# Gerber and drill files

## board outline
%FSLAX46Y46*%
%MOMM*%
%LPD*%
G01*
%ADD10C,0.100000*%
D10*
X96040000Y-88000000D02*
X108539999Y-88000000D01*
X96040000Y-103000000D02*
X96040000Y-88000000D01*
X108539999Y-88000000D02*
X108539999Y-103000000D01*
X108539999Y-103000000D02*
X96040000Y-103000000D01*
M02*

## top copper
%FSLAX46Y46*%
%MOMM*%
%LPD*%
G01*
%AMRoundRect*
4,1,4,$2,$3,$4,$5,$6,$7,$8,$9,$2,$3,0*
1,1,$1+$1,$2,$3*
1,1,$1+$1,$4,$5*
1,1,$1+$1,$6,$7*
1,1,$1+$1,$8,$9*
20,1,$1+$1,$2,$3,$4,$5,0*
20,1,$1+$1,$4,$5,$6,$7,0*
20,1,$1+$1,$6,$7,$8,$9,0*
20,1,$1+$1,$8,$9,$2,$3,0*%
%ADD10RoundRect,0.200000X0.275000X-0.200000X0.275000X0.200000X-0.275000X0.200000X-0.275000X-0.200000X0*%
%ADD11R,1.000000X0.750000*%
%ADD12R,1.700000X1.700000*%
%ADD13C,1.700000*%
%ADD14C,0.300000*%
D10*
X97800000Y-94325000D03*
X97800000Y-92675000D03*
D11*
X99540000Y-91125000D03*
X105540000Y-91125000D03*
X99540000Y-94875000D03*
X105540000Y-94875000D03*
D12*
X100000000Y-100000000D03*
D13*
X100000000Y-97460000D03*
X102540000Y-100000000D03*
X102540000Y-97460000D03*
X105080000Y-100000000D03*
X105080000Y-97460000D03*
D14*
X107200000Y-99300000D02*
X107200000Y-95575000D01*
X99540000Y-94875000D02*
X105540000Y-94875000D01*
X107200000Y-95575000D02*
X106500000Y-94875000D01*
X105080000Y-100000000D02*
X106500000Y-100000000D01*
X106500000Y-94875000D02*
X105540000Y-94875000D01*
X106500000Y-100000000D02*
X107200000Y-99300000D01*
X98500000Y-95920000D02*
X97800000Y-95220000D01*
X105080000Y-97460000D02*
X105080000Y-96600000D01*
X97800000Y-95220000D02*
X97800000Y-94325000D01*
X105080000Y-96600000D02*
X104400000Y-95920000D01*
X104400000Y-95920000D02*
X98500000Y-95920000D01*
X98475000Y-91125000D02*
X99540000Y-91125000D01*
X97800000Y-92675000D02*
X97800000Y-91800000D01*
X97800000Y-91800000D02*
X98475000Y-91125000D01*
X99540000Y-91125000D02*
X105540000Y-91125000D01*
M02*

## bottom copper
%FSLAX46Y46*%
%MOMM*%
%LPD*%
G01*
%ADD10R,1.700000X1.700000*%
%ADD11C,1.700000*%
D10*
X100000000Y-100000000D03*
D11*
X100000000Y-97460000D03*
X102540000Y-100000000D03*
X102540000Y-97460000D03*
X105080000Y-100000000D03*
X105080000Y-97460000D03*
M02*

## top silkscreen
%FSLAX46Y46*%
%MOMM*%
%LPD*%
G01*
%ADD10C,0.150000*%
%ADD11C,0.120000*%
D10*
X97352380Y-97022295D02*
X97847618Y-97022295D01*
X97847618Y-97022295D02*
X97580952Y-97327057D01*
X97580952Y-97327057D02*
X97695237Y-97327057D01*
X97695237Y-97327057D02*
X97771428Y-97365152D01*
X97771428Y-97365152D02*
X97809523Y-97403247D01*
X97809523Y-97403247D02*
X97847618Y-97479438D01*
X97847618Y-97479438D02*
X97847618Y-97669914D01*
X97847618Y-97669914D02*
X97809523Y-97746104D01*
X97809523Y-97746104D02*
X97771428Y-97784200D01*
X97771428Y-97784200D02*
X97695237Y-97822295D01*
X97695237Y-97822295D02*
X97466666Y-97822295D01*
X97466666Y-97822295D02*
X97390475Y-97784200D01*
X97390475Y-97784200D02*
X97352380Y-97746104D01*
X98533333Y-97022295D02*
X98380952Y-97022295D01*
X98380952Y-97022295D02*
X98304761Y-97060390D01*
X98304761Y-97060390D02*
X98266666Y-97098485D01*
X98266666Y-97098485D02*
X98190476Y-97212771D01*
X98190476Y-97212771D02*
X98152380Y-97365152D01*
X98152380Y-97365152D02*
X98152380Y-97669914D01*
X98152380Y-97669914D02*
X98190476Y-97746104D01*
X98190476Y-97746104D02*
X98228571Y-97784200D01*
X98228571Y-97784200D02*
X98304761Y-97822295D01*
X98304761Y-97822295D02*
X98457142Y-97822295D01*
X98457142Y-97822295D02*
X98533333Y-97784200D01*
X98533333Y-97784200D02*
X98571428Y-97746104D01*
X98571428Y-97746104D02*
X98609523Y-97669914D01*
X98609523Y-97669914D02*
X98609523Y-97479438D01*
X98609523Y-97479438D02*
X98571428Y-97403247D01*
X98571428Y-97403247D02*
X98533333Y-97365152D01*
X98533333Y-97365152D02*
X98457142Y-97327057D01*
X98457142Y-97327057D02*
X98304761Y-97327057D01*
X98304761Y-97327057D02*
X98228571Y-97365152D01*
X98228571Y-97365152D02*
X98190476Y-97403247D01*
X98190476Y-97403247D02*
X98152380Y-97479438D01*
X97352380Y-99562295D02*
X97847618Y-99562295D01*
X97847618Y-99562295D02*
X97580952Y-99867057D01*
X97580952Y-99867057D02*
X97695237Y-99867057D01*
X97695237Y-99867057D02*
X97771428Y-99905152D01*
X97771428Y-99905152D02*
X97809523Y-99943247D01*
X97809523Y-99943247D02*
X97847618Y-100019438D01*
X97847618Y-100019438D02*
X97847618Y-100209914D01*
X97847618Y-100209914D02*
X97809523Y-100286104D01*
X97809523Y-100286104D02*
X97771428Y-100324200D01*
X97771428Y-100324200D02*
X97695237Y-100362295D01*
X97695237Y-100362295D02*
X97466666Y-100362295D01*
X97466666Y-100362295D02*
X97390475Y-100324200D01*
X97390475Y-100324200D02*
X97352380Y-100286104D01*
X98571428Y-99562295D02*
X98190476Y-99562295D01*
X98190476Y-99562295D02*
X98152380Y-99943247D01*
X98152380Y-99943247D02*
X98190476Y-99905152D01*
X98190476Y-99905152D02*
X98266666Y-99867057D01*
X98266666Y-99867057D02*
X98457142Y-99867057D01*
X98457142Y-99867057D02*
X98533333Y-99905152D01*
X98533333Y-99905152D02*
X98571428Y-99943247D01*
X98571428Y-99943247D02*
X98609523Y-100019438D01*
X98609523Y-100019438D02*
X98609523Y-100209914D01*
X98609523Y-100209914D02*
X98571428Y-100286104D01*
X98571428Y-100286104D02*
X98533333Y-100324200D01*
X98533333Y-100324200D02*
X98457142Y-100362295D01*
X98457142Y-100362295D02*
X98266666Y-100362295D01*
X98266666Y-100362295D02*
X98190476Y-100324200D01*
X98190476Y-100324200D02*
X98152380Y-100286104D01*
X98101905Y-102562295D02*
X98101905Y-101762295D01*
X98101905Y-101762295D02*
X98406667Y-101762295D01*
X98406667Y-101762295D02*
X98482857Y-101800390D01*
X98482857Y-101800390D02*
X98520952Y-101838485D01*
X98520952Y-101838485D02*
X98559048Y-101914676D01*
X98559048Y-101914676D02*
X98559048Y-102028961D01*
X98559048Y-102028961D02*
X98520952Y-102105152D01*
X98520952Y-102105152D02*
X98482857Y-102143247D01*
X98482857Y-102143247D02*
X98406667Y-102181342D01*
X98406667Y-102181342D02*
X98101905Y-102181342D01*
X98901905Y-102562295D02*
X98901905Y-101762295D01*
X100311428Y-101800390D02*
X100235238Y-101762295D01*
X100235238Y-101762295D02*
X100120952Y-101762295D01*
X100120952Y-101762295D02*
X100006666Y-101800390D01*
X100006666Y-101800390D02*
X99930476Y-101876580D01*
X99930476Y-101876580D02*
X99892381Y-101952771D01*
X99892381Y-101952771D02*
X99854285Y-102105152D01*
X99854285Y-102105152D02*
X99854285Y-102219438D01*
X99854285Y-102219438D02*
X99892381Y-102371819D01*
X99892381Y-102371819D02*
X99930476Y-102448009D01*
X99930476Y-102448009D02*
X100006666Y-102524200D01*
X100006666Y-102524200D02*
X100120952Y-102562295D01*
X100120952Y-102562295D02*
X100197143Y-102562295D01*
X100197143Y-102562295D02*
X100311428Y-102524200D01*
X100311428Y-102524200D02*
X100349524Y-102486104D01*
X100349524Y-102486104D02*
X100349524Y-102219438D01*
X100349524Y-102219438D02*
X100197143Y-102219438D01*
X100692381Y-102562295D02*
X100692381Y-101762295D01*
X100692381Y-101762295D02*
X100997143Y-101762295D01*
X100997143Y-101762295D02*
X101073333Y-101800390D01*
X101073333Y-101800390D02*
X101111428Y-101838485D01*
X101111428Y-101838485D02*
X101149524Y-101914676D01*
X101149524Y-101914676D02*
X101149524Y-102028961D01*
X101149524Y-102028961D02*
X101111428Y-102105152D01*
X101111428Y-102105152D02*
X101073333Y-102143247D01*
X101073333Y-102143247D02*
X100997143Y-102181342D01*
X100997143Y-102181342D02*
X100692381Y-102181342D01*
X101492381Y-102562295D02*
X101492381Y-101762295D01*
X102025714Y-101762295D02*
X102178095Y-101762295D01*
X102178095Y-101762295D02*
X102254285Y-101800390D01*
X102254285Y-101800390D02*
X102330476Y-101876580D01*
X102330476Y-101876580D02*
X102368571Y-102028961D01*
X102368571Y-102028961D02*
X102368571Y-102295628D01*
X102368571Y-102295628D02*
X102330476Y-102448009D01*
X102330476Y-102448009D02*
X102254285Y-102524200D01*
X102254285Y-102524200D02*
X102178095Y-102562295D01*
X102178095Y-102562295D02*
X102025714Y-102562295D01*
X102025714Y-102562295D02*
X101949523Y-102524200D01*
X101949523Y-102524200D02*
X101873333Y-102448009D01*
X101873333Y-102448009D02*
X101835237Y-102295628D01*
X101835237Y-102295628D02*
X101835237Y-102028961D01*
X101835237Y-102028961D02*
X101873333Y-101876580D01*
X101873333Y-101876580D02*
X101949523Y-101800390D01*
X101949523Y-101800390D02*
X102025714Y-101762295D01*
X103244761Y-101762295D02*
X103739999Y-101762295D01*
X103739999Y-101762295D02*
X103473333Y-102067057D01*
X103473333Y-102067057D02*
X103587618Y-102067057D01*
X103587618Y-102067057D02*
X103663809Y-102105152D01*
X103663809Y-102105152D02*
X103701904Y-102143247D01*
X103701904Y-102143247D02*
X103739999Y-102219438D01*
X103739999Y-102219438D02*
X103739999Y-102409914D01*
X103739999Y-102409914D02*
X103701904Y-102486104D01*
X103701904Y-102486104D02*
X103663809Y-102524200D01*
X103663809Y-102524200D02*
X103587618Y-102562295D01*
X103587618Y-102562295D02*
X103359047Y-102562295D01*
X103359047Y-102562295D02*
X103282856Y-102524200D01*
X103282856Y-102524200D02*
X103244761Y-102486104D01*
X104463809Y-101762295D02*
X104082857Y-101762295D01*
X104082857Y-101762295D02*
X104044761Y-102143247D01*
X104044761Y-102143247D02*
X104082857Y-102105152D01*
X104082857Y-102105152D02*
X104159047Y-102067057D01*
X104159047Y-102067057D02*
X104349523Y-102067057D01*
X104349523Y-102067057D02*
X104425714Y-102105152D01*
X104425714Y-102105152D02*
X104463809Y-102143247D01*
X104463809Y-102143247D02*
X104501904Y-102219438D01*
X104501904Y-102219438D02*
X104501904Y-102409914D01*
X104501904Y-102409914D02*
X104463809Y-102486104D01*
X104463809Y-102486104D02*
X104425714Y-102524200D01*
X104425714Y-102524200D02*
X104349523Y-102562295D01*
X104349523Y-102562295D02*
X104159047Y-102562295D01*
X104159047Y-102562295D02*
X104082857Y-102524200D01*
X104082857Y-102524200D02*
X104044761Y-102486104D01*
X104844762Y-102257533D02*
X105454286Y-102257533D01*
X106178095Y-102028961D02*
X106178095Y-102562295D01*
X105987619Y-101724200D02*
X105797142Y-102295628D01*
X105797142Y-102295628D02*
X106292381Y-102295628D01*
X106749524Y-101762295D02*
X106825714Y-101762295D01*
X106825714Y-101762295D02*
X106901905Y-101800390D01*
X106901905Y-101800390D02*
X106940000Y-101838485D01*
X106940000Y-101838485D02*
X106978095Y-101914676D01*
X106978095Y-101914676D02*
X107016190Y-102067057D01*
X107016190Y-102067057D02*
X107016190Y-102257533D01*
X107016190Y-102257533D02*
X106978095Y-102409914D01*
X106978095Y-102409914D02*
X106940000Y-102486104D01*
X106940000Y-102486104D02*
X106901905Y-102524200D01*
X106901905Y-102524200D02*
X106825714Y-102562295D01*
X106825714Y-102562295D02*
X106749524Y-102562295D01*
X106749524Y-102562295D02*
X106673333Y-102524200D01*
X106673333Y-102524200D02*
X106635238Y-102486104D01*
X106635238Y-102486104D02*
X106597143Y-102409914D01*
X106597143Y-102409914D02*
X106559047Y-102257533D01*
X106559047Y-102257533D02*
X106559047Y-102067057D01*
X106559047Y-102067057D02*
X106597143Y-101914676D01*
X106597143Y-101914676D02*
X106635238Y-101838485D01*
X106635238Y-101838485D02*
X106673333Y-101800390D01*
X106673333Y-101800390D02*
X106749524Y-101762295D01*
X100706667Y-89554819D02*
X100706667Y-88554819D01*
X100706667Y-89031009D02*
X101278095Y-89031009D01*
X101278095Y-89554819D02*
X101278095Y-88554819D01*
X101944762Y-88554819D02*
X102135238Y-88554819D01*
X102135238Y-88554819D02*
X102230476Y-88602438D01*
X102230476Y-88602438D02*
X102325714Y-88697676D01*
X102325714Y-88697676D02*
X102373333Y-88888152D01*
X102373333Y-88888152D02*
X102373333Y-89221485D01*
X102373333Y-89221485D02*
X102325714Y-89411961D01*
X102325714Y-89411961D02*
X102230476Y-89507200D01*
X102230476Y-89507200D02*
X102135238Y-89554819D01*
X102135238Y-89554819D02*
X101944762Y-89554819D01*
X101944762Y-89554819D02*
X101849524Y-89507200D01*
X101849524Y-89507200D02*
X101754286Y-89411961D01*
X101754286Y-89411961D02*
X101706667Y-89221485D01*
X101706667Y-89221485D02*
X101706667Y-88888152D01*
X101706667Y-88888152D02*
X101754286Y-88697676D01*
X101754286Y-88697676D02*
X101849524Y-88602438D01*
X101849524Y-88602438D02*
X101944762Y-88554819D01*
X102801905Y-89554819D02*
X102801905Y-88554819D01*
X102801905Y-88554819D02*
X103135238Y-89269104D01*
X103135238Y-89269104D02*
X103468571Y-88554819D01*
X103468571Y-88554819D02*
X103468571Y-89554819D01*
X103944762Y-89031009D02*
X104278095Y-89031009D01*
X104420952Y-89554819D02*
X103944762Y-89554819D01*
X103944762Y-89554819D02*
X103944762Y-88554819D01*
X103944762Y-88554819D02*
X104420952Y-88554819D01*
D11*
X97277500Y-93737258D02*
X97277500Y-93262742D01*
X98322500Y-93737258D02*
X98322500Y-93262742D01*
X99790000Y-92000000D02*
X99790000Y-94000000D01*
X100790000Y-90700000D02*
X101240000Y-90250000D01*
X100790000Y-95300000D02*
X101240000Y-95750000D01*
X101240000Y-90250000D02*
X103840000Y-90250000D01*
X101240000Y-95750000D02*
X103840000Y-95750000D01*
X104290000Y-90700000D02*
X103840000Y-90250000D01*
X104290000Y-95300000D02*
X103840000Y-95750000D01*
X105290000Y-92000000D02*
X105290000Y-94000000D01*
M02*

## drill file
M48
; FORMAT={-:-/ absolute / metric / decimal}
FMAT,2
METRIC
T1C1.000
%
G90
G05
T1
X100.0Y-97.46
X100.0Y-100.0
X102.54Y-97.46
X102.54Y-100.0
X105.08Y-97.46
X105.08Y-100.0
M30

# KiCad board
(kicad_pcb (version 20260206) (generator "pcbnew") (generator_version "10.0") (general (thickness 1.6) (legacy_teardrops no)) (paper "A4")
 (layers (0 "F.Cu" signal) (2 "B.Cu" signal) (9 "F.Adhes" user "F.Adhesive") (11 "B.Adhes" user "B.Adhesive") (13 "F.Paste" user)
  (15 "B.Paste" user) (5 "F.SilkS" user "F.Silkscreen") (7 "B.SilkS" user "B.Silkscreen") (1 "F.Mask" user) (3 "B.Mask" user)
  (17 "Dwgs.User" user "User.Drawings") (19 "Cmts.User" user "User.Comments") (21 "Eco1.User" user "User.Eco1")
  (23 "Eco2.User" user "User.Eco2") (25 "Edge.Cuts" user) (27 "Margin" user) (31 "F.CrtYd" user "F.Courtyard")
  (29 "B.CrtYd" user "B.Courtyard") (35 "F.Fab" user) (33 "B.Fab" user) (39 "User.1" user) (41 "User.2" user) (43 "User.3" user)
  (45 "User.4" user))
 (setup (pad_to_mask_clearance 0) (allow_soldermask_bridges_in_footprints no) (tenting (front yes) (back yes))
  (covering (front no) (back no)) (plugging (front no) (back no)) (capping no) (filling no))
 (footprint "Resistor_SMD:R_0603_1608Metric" (layer "F.Cu") (at 97.8 93.5 90)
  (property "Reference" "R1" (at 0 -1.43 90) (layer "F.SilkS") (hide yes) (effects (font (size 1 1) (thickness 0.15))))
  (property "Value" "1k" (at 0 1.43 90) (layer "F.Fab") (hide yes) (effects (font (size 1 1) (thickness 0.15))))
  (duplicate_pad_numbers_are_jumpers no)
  (fp_line (start -0.237258 -0.5225) (end 0.237258 -0.5225) (stroke (width 0.12) (type solid)) (layer "F.SilkS"))
  (fp_line (start -0.237258 0.5225) (end 0.237258 0.5225) (stroke (width 0.12) (type solid)) (layer "F.SilkS"))
  (pad "1" smd roundrect (at -0.825 0 90) (size 0.8 0.95) (layers "F.Cu" "F.Mask" "F.Paste") (roundrect_rratio 0.25) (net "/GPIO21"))
  (pad "2" smd roundrect (at 0.825 0 90) (size 0.8 0.95) (layers "F.Cu" "F.Mask" "F.Paste") (roundrect_rratio 0.25) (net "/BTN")))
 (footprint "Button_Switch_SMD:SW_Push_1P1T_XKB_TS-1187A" (layer "F.Cu") (at 102.54 93)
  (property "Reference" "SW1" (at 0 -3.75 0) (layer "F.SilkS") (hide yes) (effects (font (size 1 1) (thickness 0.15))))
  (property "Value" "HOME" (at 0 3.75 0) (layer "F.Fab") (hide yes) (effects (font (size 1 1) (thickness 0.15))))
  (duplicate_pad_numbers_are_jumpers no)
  (fp_line (start -2.75 -1) (end -2.75 1) (stroke (width 0.12) (type solid)) (layer "F.SilkS"))
  (fp_line (start -1.75 -2.3) (end -1.3 -2.75) (stroke (width 0.12) (type solid)) (layer "F.SilkS"))
  (fp_line (start -1.75 2.3) (end -1.3 2.75) (stroke (width 0.12) (type solid)) (layer "F.SilkS"))
  (fp_line (start -1.3 -2.75) (end 1.3 -2.75) (stroke (width 0.12) (type solid)) (layer "F.SilkS"))
  (fp_line (start -1.3 2.75) (end 1.3 2.75) (stroke (width 0.12) (type solid)) (layer "F.SilkS"))
  (fp_line (start 1.75 -2.3) (end 1.3 -2.75) (stroke (width 0.12) (type solid)) (layer "F.SilkS"))
  (fp_line (start 1.75 2.3) (end 1.3 2.75) (stroke (width 0.12) (type solid)) (layer "F.SilkS"))
  (fp_line (start 2.75 -1) (end 2.75 1) (stroke (width 0.12) (type solid)) (layer "F.SilkS"))
  (pad "1" smd rect (at -3 -1.875) (size 1 0.75) (layers "F.Cu" "F.Mask" "F.Paste") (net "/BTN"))
  (pad "1" smd rect (at 3 -1.875) (size 1 0.75) (layers "F.Cu" "F.Mask" "F.Paste") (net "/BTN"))
  (pad "2" smd rect (at -3 1.875) (size 1 0.75) (layers "F.Cu" "F.Mask" "F.Paste") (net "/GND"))
  (pad "2" smd rect (at 3 1.875) (size 1 0.75) (layers "F.Cu" "F.Mask" "F.Paste") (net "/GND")))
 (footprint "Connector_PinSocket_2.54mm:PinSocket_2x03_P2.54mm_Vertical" (layer "B.Cu") (at 100 100 -90)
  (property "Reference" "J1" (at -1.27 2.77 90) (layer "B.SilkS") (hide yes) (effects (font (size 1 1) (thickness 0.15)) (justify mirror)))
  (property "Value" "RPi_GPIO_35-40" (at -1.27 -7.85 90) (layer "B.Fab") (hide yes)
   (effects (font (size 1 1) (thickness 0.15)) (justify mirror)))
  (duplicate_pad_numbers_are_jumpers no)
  (pad "1" thru_hole rect (at 0 0 270) (size 1.7 1.7) (drill 1) (layers "*.Cu" "*.Mask") (remove_unused_layers no)
   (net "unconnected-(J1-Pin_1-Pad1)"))
  (pad "2" thru_hole circle (at -2.54 0 270) (size 1.7 1.7) (drill 1) (layers "*.Cu" "*.Mask") (remove_unused_layers no)
   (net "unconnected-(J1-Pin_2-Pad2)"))
  (pad "3" thru_hole circle (at 0 -2.54 270) (size 1.7 1.7) (drill 1) (layers "*.Cu" "*.Mask") (remove_unused_layers no)
   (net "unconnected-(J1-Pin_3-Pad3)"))
  (pad "4" thru_hole circle (at -2.54 -2.54 270) (size 1.7 1.7) (drill 1) (layers "*.Cu" "*.Mask") (remove_unused_layers no)
   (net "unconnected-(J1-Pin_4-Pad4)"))
  (pad "5" thru_hole circle (at 0 -5.08 270) (size 1.7 1.7) (drill 1) (layers "*.Cu" "*.Mask") (remove_unused_layers no) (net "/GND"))
  (pad "6" thru_hole circle (at -2.54 -5.08 270) (size 1.7 1.7) (drill 1) (layers "*.Cu" "*.Mask") (remove_unused_layers no) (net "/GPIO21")))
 (gr_line (start 96.04 88) (end 108.539999 88) (stroke (width 0.1) (type default)) (layer "Edge.Cuts"))
 (gr_line (start 96.04 103) (end 96.04 88) (stroke (width 0.1) (type default)) (layer "Edge.Cuts"))
 (gr_line (start 108.539999 88) (end 108.539999 103) (stroke (width 0.1) (type default)) (layer "Edge.Cuts"))
 (gr_line (start 108.539999 103) (end 96.04 103) (stroke (width 0.1) (type default)) (layer "Edge.Cuts"))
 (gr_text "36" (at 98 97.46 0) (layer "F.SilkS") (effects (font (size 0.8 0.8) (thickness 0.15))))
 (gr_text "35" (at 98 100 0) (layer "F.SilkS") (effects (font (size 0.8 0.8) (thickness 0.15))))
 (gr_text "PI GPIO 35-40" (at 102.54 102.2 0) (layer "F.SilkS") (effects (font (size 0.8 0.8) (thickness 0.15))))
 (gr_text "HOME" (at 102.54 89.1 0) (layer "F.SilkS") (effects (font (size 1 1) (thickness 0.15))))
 (segment (start 107.2 99.3) (end 107.2 95.575) (width 0.3) (layer "F.Cu") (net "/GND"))
 (segment (start 99.54 94.875) (end 105.54 94.875) (width 0.3) (layer "F.Cu") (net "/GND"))
 (segment (start 107.2 95.575) (end 106.5 94.875) (width 0.3) (layer "F.Cu") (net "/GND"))
 (segment (start 105.08 100) (end 106.5 100) (width 0.3) (layer "F.Cu") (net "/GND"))
 (segment (start 106.5 94.875) (end 105.54 94.875) (width 0.3) (layer "F.Cu") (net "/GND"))
 (segment (start 106.5 100) (end 107.2 99.3) (width 0.3) (layer "F.Cu") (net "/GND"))
 (segment (start 98.5 95.92) (end 97.8 95.22) (width 0.3) (layer "F.Cu") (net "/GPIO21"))
 (segment (start 105.08 97.46) (end 105.08 96.6) (width 0.3) (layer "F.Cu") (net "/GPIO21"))
 (segment (start 97.8 95.22) (end 97.8 94.325) (width 0.3) (layer "F.Cu") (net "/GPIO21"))
 (segment (start 105.08 96.6) (end 104.4 95.92) (width 0.3) (layer "F.Cu") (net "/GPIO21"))
 (segment (start 104.4 95.92) (end 98.5 95.92) (width 0.3) (layer "F.Cu") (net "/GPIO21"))
 (segment (start 98.475 91.125) (end 99.54 91.125) (width 0.3) (layer "F.Cu") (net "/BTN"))
 (segment (start 97.8 92.675) (end 97.8 91.8) (width 0.3) (layer "F.Cu") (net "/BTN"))
 (segment (start 97.8 91.8) (end 98.475 91.125) (width 0.3) (layer "F.Cu") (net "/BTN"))
 (segment (start 99.54 91.125) (end 105.54 91.125) (width 0.3) (layer "F.Cu") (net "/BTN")))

